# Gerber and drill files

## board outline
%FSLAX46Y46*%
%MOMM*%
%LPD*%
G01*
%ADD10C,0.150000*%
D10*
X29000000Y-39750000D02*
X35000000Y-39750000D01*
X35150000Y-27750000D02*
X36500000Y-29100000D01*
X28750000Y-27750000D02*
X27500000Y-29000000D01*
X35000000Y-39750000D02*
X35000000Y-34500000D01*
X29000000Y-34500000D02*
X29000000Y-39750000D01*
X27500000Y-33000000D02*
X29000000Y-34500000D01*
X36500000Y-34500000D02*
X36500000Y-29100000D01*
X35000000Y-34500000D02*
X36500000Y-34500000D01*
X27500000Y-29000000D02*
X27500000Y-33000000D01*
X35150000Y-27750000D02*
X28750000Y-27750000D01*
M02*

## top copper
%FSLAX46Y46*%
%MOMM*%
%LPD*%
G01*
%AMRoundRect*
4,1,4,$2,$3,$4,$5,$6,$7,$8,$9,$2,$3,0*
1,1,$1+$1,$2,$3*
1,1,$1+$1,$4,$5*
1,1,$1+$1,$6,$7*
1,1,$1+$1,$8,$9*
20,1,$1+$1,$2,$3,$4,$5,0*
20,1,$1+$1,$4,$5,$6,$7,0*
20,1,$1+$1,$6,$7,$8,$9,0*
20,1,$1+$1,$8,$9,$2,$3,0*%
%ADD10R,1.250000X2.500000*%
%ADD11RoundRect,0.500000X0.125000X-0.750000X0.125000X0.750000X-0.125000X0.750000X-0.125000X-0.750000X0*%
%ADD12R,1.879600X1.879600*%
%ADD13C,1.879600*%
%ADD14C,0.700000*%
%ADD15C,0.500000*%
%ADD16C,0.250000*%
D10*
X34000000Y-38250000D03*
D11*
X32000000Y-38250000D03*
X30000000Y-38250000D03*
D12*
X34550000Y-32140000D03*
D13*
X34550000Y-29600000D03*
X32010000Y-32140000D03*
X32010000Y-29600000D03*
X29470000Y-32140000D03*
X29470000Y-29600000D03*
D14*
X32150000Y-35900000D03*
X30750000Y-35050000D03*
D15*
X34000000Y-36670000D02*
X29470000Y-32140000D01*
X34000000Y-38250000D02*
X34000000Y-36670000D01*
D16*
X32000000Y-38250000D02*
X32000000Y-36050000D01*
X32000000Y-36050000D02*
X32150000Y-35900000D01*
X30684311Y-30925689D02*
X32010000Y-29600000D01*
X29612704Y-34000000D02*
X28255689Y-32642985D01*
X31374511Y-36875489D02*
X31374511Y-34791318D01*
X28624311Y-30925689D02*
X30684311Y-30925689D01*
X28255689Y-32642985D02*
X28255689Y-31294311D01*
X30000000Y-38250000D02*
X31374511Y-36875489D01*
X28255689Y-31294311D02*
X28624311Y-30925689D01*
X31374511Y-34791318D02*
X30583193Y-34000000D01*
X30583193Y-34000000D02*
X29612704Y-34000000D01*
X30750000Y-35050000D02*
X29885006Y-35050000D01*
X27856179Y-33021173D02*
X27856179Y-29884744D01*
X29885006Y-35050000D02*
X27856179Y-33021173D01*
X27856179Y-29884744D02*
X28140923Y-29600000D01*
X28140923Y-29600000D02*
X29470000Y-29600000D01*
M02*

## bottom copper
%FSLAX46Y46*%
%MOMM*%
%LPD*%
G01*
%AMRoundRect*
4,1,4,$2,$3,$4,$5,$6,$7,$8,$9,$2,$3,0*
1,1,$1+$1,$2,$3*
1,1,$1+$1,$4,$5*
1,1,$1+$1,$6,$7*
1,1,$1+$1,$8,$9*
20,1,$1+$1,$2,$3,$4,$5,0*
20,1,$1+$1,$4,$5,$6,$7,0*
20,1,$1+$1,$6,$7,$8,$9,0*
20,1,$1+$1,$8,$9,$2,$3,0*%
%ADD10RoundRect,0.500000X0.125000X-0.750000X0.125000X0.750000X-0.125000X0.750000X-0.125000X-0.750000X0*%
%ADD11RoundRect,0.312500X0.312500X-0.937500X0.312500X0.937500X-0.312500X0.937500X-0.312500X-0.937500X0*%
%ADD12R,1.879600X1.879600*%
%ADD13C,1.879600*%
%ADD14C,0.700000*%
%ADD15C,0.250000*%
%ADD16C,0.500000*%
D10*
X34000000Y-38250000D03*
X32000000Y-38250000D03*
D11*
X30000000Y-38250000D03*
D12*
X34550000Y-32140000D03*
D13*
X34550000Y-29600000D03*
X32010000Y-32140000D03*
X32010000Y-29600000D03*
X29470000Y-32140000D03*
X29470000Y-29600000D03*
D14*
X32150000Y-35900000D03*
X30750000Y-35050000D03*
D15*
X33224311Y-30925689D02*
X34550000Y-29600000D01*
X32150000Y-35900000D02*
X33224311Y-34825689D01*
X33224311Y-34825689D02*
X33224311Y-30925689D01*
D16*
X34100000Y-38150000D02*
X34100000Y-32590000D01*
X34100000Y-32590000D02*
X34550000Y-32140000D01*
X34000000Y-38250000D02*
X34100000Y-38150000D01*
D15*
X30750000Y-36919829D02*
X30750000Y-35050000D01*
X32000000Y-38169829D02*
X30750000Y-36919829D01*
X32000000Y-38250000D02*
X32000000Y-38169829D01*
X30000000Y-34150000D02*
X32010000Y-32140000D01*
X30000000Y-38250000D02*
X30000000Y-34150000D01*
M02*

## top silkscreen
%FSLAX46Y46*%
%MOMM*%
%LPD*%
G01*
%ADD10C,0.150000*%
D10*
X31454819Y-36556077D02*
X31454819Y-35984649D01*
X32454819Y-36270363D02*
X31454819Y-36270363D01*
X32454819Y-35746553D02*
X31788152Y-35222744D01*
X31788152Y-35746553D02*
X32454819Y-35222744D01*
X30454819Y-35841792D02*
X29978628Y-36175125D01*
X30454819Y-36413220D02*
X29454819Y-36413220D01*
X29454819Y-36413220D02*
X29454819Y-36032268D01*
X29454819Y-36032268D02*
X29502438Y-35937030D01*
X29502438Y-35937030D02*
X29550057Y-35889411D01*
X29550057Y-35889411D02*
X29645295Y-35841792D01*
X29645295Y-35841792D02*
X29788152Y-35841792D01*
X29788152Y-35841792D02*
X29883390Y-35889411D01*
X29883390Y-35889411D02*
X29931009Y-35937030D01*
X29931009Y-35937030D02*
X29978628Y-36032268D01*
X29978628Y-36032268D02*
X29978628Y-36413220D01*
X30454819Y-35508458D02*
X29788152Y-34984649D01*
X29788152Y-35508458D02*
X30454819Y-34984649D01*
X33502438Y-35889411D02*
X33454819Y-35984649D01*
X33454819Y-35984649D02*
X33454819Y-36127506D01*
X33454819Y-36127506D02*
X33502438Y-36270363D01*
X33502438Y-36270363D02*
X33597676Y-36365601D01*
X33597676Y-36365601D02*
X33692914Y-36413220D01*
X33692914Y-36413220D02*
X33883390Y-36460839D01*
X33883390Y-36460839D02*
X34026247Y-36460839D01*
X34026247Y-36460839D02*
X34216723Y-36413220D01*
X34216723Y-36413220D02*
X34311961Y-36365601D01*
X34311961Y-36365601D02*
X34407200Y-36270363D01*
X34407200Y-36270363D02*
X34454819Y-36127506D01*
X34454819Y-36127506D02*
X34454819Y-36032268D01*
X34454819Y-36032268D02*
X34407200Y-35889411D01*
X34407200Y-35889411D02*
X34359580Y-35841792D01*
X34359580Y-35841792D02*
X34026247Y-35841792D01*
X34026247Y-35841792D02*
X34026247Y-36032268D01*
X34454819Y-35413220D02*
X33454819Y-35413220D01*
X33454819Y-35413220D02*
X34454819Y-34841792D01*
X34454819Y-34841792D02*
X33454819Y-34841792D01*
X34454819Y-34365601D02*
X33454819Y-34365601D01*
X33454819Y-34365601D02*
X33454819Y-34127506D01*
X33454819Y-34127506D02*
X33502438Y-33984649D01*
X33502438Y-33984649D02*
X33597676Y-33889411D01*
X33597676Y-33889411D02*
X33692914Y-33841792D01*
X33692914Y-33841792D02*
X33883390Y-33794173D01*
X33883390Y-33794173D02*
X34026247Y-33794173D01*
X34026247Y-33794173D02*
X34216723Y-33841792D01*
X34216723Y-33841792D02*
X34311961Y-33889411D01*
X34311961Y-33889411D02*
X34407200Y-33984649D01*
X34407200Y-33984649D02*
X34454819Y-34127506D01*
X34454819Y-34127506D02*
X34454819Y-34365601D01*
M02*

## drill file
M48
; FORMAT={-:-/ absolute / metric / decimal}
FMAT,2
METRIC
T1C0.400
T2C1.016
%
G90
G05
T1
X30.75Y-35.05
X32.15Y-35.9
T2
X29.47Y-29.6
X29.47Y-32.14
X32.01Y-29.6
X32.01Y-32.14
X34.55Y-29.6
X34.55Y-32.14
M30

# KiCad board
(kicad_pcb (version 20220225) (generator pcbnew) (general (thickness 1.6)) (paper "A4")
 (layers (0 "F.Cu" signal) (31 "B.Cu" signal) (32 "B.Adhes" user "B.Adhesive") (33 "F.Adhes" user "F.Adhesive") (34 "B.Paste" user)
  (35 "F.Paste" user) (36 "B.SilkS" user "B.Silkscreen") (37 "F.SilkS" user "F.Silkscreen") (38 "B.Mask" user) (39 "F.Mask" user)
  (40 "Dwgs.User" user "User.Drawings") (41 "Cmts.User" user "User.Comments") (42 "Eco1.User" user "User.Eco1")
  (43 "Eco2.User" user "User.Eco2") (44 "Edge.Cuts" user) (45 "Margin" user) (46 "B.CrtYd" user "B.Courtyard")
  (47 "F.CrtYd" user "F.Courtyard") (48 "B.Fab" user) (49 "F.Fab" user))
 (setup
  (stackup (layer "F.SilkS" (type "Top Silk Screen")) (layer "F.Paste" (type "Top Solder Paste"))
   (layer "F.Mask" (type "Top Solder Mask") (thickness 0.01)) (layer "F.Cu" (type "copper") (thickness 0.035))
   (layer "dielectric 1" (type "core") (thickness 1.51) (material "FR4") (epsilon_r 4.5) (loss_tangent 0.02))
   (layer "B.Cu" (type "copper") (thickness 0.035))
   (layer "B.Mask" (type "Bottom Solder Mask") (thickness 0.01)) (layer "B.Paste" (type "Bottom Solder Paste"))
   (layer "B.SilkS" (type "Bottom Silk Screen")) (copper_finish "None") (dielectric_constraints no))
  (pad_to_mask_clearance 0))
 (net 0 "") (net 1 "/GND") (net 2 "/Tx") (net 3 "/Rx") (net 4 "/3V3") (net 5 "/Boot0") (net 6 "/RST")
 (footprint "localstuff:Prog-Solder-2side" (layer "F.Cu") (at 32 38.25 90)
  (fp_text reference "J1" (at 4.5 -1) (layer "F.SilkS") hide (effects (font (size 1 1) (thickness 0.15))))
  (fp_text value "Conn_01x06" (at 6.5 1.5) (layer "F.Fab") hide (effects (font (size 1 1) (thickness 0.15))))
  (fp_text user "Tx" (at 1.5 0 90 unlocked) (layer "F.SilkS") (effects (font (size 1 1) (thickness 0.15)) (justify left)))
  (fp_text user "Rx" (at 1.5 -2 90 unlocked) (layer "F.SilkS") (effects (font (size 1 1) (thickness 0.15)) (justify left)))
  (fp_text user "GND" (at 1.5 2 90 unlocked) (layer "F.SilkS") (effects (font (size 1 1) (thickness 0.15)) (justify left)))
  (pad "1" smd rect (at 0 2 90) (size 2.5 1.25) (layers "F.Cu" "F.Mask") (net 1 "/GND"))
  (pad "2" smd roundrect (at 0 0 90) (size 2.5 1.25) (layers "F.Cu" "F.Mask") (roundrect_rratio 0.4) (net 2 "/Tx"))
  (pad "3" smd roundrect (at 0 -2 90) (size 2.5 1.25) (layers "F.Cu" "F.Mask") (roundrect_rratio 0.4) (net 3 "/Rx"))
  (pad "4" smd roundrect (at 0 2 90) (size 2.5 1.25) (layers "B.Cu" "B.Mask") (roundrect_rratio 0.4) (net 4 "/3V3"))
  (pad "5" smd roundrect (at 0 0 90) (size 2.5 1.25) (layers "B.Cu" "B.Mask") (roundrect_rratio 0.4) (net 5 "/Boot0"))
  (pad "6" smd roundrect (at 0 -2 90) (size 2.5 1.25) (layers "B.Cu" "B.Mask") (roundrect_rratio 0.25) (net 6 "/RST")))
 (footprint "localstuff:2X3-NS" (layer "B.Cu") (at 32.01 30.87 180)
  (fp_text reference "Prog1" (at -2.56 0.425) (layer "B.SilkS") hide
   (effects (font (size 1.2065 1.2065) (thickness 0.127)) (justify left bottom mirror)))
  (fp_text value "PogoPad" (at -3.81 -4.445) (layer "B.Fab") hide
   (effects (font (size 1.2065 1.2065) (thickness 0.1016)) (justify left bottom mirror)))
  (pad "1" thru_hole rect locked (at -2.54 -1.27 180) (size 1.8796 1.8796) (drill 1.016) (layers *.Cu *.Mask) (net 4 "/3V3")
   (solder_mask_margin 0.1016))
  (pad "2" thru_hole circle locked (at -2.54 1.27 180) (size 1.8796 1.8796) (drill 1.016) (layers *.Cu *.Mask) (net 2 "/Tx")
   (solder_mask_margin 0.1016))
  (pad "3" thru_hole circle locked (at 0 -1.27 180) (size 1.8796 1.8796) (drill 1.016) (layers *.Cu *.Mask) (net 6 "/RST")
   (solder_mask_margin 0.1016))
  (pad "4" thru_hole circle locked (at 0 1.27 180) (size 1.8796 1.8796) (drill 1.016) (layers *.Cu *.Mask) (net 3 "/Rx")
   (solder_mask_margin 0.1016))
  (pad "5" thru_hole circle locked (at 2.54 -1.27 180) (size 1.8796 1.8796) (drill 1.016) (layers *.Cu *.Mask) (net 1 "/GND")
   (solder_mask_margin 0.1016))
  (pad "6" thru_hole circle locked (at 2.54 1.27 180) (size 1.8796 1.8796) (drill 1.016) (layers *.Cu *.Mask) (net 5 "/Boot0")
   (solder_mask_margin 0.1016)))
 (gr_line (start 29 39.75) (end 35 39.75) (stroke (width 0.15) (type solid)) (layer "Edge.Cuts"))
 (gr_line (start 35.15 27.75) (end 36.5 29.1) (stroke (width 0.15) (type solid)) (layer "Edge.Cuts"))
 (gr_line (start 28.75 27.75) (end 27.5 29) (stroke (width 0.15) (type solid)) (layer "Edge.Cuts"))
 (gr_line (start 35 39.75) (end 35 34.5) (stroke (width 0.15) (type solid)) (layer "Edge.Cuts"))
 (gr_line (start 29 34.5) (end 29 39.75) (stroke (width 0.15) (type solid)) (layer "Edge.Cuts"))
 (gr_line (start 27.5 33) (end 29 34.5) (stroke (width 0.15) (type solid)) (layer "Edge.Cuts"))
 (gr_line (start 36.5 34.5) (end 36.5 29.1) (stroke (width 0.15) (type solid)) (layer "Edge.Cuts"))
 (gr_line (start 35 34.5) (end 36.5 34.5) (stroke (width 0.15) (type solid)) (layer "Edge.Cuts"))
 (gr_line (start 27.5 29) (end 27.5 33) (stroke (width 0.15) (type solid)) (layer "Edge.Cuts"))
 (gr_line (start 35.15 27.75) (end 28.75 27.75) (stroke (width 0.15) (type solid)) (layer "Edge.Cuts"))
 (segment (start 34 36.67) (end 29.47 32.14) (width 0.5) (layer "F.Cu") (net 1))
 (segment (start 34 38.25) (end 34 36.67) (width 0.5) (layer "F.Cu") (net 1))
 (segment (start 32 38.25) (end 32 36.05) (width 0.25) (layer "F.Cu") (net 2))
 (segment (start 32 36.05) (end 32.15 35.9) (width 0.25) (layer "F.Cu") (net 2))
 (via (at 32.15 35.9) (size 0.7) (drill 0.4) (layers "F.Cu" "B.Cu") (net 2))
 (segment (start 33.224311 30.925689) (end 34.55 29.6) (width 0.25) (layer "B.Cu") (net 2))
 (segment (start 32.15 35.9) (end 33.224311 34.825689) (width 0.25) (layer "B.Cu") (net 2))
 (segment (start 33.224311 34.825689) (end 33.224311 30.925689) (width 0.25) (layer "B.Cu") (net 2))
 (segment (start 30.684311 30.925689) (end 32.01 29.6) (width 0.25) (layer "F.Cu") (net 3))
 (segment (start 29.612704 34) (end 28.255689 32.642985) (width 0.25) (layer "F.Cu") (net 3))
 (segment (start 31.374511 36.875489) (end 31.374511 34.791318) (width 0.25) (layer "F.Cu") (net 3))
 (segment (start 28.624311 30.925689) (end 30.684311 30.925689) (width 0.25) (layer "F.Cu") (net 3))
 (segment (start 28.255689 32.642985) (end 28.255689 31.294311) (width 0.25) (layer "F.Cu") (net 3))
 (segment (start 30 38.25) (end 31.374511 36.875489) (width 0.25) (layer "F.Cu") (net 3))
 (segment (start 28.255689 31.294311) (end 28.624311 30.925689) (width 0.25) (layer "F.Cu") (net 3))
 (segment (start 31.374511 34.791318) (end 30.583193 34) (width 0.25) (layer "F.Cu") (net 3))
 (segment (start 30.583193 34) (end 29.612704 34) (width 0.25) (layer "F.Cu") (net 3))
 (segment (start 34.1 38.15) (end 34.1 32.59) (width 0.5) (layer "B.Cu") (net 4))
 (segment (start 34.1 32.59) (end 34.55 32.14) (width 0.5) (layer "B.Cu") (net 4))
 (segment (start 34 38.25) (end 34.1 38.15) (width 0.5) (layer "B.Cu") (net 4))
 (segment (start 30.75 35.05) (end 29.885006 35.05) (width 0.25) (layer "F.Cu") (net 5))
 (segment (start 27.856179 33.021173) (end 27.856179 29.884744) (width 0.25) (layer "F.Cu") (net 5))
 (segment (start 29.885006 35.05) (end 27.856179 33.021173) (width 0.25) (layer "F.Cu") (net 5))
 (segment (start 27.856179 29.884744) (end 28.140923 29.6) (width 0.25) (layer "F.Cu") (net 5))
 (segment (start 28.140923 29.6) (end 29.47 29.6) (width 0.25) (layer "F.Cu") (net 5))
 (via (at 30.75 35.05) (size 0.7) (drill 0.4) (layers "F.Cu" "B.Cu") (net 5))
 (segment (start 30.75 36.919829) (end 30.75 35.05) (width 0.25) (layer "B.Cu") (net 5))
 (segment (start 32 38.169829) (end 30.75 36.919829) (width 0.25) (layer "B.Cu") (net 5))
 (segment (start 32 38.25) (end 32 38.169829) (width 0.25) (layer "B.Cu") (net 5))
 (segment (start 30 34.15) (end 32.01 32.14) (width 0.25) (layer "B.Cu") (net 6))
 (segment (start 30 38.25) (end 30 34.15) (width 0.25) (layer "B.Cu") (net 6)))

